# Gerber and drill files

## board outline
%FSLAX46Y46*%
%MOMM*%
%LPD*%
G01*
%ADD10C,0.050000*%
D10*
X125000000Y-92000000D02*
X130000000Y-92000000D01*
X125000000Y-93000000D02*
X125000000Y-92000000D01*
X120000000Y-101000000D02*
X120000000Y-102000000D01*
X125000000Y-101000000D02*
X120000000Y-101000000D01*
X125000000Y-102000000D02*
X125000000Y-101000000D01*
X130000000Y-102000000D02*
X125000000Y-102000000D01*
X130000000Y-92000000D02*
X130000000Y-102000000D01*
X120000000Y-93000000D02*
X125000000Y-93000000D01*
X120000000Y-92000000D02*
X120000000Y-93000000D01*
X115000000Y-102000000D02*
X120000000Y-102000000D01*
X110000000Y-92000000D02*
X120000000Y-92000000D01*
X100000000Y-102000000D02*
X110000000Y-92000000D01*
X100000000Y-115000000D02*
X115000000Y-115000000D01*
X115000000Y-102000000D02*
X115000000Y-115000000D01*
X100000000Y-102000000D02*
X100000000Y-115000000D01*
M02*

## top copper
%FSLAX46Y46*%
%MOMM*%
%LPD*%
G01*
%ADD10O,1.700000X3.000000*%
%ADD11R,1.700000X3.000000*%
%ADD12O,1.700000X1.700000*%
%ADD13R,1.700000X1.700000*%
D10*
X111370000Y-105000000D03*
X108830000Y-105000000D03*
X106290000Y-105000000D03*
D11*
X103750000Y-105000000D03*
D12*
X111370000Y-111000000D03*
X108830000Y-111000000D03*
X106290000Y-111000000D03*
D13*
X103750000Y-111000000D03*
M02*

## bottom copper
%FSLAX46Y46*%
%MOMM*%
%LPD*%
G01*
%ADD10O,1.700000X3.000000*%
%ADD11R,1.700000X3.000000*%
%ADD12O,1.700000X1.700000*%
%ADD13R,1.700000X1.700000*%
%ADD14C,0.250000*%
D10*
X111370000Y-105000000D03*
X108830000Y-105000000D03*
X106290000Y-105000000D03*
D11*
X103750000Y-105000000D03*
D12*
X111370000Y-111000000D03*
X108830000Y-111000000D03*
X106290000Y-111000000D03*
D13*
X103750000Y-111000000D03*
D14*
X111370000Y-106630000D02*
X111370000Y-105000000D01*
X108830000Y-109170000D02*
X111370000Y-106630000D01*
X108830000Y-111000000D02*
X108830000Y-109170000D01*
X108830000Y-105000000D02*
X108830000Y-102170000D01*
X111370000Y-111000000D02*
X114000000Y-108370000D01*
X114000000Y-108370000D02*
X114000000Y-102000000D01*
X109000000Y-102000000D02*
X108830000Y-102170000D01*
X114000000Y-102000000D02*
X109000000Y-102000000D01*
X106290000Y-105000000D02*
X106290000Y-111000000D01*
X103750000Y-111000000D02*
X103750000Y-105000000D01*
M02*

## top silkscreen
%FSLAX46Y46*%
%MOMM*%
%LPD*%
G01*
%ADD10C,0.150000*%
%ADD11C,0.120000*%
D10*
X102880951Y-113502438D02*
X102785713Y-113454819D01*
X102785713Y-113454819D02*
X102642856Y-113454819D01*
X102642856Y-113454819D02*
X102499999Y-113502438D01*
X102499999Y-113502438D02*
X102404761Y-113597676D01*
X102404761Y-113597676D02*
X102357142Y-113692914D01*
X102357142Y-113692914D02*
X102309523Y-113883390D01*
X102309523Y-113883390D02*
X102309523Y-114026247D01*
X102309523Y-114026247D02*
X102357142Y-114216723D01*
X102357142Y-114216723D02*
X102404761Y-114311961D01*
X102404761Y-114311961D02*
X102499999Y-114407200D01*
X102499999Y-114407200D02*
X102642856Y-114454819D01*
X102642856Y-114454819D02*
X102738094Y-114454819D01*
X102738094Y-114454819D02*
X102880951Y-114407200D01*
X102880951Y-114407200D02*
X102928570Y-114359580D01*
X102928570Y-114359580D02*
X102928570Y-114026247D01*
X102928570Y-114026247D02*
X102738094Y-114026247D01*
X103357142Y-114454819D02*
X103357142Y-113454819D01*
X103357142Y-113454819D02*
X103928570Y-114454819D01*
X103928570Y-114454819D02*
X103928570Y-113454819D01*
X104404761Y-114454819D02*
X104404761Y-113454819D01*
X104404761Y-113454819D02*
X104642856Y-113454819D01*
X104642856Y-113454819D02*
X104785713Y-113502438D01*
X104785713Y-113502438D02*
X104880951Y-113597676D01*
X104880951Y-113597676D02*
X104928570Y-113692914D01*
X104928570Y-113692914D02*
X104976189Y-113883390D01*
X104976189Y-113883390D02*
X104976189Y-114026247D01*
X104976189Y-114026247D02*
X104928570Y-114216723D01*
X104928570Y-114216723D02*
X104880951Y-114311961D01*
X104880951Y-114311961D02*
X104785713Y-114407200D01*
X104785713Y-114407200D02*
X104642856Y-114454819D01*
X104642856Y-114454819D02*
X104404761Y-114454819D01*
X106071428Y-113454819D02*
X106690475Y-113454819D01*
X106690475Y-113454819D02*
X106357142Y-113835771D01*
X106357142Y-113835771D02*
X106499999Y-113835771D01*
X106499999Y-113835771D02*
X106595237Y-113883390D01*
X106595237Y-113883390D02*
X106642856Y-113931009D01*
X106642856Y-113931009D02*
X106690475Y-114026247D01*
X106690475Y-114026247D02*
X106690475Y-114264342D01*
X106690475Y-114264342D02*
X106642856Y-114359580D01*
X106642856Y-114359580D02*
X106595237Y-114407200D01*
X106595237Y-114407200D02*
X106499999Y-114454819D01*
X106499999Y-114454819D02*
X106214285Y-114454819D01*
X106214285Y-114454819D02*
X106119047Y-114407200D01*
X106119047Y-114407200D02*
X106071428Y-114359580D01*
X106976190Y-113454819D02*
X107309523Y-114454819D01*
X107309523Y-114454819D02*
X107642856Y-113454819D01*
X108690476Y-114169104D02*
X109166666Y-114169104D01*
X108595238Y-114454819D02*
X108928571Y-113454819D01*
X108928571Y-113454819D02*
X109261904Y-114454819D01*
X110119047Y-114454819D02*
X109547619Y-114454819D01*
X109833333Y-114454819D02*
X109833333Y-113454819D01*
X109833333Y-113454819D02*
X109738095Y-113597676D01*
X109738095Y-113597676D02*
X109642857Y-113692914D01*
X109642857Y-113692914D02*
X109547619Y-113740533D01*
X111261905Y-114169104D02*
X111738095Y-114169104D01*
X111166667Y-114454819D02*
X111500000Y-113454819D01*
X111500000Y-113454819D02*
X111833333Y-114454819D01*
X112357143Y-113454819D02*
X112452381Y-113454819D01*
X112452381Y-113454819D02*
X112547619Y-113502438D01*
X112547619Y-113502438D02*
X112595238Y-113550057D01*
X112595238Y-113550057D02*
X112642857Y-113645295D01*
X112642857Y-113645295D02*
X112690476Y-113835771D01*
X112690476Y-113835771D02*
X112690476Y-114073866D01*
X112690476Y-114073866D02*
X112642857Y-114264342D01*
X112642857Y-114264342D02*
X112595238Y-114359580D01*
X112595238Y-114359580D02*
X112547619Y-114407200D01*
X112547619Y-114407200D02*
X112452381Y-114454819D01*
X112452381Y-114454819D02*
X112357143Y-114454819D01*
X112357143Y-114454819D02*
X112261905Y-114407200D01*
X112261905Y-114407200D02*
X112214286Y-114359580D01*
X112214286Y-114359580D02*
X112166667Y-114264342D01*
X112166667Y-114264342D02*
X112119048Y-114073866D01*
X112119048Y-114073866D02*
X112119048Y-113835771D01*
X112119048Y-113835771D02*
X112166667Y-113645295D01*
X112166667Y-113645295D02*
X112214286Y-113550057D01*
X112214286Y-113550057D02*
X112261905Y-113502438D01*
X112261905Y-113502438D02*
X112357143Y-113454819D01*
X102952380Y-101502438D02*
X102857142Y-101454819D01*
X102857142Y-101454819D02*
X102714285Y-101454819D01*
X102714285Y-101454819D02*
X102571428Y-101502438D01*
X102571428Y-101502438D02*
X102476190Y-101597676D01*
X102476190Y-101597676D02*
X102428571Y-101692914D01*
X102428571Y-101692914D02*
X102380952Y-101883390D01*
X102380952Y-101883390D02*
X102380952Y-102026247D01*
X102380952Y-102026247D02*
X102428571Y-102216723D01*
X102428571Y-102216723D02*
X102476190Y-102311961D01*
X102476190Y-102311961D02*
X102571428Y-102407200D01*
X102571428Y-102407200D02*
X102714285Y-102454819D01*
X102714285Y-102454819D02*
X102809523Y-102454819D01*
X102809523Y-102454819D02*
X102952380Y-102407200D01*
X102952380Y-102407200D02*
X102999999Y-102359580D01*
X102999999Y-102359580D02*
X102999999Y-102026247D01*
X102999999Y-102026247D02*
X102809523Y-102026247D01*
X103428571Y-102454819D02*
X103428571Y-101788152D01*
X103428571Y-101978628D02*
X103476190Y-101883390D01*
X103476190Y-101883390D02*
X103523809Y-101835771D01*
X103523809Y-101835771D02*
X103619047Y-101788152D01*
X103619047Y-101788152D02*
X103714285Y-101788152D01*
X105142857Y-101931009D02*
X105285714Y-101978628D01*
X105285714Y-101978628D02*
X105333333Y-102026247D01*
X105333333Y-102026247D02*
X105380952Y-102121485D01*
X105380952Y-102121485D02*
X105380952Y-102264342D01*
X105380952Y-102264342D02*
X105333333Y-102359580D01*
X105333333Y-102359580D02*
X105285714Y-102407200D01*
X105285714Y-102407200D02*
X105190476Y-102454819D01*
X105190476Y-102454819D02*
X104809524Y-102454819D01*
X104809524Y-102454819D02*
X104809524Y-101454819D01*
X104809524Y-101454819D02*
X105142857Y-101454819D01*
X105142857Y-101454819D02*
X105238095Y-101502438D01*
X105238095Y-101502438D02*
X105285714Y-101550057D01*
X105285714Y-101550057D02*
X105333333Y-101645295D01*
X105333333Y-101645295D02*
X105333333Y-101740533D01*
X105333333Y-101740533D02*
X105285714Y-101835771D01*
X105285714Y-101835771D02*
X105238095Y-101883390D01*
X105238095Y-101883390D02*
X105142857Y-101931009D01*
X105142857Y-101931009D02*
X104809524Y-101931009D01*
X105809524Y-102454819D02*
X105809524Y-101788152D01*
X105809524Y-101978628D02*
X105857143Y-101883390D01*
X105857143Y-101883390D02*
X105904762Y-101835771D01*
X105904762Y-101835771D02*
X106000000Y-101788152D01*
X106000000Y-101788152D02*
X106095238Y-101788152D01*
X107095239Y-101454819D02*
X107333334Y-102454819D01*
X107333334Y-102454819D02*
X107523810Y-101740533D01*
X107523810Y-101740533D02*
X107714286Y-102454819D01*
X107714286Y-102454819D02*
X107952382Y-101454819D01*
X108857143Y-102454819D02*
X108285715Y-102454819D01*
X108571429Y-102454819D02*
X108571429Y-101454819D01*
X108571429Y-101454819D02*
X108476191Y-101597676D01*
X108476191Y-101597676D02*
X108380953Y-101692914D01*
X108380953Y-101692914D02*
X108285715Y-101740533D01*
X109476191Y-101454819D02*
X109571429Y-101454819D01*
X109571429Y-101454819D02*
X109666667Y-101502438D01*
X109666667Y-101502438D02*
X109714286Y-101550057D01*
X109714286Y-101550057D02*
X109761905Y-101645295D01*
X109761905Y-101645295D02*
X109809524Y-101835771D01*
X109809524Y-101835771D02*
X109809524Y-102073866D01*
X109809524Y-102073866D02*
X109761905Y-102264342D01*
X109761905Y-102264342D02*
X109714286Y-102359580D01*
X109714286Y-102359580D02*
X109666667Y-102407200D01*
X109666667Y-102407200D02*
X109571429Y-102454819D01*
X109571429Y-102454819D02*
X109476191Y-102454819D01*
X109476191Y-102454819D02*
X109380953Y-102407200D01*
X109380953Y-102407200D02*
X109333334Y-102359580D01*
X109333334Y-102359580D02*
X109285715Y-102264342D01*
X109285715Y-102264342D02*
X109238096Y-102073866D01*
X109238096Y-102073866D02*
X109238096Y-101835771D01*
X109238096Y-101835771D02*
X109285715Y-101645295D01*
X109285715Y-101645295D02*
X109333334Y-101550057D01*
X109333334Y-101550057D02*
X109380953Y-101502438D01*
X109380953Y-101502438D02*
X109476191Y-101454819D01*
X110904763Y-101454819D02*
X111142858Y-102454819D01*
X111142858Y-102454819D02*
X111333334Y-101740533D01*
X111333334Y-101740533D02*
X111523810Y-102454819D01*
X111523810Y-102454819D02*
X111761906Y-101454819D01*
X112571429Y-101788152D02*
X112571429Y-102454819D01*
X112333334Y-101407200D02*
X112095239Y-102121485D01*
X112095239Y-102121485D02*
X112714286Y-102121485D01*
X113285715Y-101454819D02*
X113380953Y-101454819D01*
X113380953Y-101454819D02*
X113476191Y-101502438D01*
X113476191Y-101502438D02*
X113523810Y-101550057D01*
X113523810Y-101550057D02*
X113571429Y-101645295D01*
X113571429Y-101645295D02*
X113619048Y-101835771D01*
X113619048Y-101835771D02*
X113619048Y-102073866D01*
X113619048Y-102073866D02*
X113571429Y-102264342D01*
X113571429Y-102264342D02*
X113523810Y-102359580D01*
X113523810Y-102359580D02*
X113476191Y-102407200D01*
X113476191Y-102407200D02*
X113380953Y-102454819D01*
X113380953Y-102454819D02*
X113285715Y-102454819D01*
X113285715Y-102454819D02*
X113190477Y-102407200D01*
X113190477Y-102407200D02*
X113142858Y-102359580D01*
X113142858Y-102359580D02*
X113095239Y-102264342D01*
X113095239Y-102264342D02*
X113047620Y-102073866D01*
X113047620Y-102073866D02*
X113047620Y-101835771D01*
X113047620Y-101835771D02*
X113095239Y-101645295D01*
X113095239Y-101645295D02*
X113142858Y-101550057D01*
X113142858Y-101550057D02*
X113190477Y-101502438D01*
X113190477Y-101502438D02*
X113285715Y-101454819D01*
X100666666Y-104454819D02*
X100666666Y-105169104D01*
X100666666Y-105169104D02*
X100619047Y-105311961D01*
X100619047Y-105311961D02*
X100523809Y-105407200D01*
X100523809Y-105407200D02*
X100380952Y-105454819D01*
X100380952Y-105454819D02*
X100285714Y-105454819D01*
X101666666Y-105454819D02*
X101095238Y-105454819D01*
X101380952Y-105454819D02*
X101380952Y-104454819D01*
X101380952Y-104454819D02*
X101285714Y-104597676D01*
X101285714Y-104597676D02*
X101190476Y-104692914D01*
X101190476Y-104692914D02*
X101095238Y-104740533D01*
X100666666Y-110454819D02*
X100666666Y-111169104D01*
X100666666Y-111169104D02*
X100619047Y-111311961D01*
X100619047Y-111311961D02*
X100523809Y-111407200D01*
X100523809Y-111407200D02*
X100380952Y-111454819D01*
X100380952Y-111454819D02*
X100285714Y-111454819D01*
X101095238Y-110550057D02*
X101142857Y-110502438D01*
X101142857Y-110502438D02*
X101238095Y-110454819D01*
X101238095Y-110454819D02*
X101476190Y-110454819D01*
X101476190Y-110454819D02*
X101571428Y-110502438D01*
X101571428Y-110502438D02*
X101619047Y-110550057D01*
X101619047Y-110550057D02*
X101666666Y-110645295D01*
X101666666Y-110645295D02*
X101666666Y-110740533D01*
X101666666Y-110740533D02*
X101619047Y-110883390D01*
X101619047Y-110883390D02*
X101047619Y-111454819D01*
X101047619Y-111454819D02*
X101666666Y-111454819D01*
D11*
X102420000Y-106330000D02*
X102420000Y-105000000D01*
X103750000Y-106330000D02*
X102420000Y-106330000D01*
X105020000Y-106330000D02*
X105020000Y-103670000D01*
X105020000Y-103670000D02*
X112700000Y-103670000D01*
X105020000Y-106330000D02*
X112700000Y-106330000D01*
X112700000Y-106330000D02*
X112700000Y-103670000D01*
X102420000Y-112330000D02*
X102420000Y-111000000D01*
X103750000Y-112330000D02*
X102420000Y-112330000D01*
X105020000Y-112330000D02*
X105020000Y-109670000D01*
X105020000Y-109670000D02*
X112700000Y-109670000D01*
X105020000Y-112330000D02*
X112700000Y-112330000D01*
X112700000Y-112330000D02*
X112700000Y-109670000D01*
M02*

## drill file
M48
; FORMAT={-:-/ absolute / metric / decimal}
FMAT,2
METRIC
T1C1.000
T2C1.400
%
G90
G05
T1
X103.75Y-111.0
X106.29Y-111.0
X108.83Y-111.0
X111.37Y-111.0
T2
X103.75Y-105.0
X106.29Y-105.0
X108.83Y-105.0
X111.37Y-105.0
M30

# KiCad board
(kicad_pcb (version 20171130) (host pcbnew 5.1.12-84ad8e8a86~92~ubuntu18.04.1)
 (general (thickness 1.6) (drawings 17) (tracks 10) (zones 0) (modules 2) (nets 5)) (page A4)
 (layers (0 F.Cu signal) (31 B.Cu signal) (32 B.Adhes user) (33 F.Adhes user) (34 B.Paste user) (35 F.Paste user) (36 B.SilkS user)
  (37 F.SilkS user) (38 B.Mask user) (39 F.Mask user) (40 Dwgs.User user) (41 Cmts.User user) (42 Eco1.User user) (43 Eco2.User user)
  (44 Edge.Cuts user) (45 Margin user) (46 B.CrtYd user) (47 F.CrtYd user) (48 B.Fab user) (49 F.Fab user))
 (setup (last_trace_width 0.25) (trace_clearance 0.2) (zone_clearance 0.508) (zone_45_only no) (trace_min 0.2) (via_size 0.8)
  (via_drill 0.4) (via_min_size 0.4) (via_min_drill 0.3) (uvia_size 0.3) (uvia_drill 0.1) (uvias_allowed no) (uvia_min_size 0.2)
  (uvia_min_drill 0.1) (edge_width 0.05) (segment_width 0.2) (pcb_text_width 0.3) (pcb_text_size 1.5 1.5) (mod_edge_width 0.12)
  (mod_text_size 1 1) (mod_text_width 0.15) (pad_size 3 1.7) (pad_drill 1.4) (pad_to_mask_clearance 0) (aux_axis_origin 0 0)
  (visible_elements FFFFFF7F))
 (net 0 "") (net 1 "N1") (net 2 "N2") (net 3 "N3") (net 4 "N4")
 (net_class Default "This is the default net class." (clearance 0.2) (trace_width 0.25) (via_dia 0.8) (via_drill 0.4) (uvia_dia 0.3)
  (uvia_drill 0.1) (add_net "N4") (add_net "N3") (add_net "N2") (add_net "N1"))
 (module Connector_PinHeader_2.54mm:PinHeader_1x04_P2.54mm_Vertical (layer F.Cu) (at 103.75 105 90)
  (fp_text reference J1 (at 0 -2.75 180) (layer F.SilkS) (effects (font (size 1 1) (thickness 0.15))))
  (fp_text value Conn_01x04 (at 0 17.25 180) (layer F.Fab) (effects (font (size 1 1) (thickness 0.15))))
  (fp_line (start -1.33 -1.33) (end 0 -1.33) (layer F.SilkS) (width 0.12))
  (fp_line (start -1.33 0) (end -1.33 -1.33) (layer F.SilkS) (width 0.12))
  (fp_line (start -1.33 1.27) (end 1.33 1.27) (layer F.SilkS) (width 0.12))
  (fp_line (start 1.33 1.27) (end 1.33 8.95) (layer F.SilkS) (width 0.12))
  (fp_line (start -1.33 1.27) (end -1.33 8.95) (layer F.SilkS) (width 0.12))
  (fp_line (start -1.33 8.95) (end 1.33 8.95) (layer F.SilkS) (width 0.12))
  (pad 4 thru_hole oval (at 0 7.62 90) (size 3 1.7) (drill 1.4) (layers *.Cu *.Mask) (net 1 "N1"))
  (pad 3 thru_hole oval (at 0 5.08 90) (size 3 1.7) (drill 1.4) (layers *.Cu *.Mask) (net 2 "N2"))
  (pad 2 thru_hole oval (at 0 2.54 90) (size 3 1.7) (drill 1.4) (layers *.Cu *.Mask) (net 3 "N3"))
  (pad 1 thru_hole rect (at 0 0 90) (size 3 1.7) (drill 1.4) (layers *.Cu *.Mask) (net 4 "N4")))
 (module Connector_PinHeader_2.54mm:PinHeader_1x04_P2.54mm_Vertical (layer F.Cu) (at 103.75 111 90)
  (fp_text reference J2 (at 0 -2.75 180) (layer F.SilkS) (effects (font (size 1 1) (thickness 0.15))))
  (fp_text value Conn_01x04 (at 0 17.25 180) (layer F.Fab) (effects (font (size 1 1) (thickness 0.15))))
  (fp_line (start -1.33 -1.33) (end 0 -1.33) (layer F.SilkS) (width 0.12))
  (fp_line (start -1.33 0) (end -1.33 -1.33) (layer F.SilkS) (width 0.12))
  (fp_line (start -1.33 1.27) (end 1.33 1.27) (layer F.SilkS) (width 0.12))
  (fp_line (start 1.33 1.27) (end 1.33 8.95) (layer F.SilkS) (width 0.12))
  (fp_line (start -1.33 1.27) (end -1.33 8.95) (layer F.SilkS) (width 0.12))
  (fp_line (start -1.33 8.95) (end 1.33 8.95) (layer F.SilkS) (width 0.12))
  (pad 4 thru_hole oval (at 0 7.62 90) (size 1.7 1.7) (drill 1) (layers *.Cu *.Mask) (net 2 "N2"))
  (pad 3 thru_hole oval (at 0 5.08 90) (size 1.7 1.7) (drill 1) (layers *.Cu *.Mask) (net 1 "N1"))
  (pad 2 thru_hole oval (at 0 2.54 90) (size 1.7 1.7) (drill 1) (layers *.Cu *.Mask) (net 3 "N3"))
  (pad 1 thru_hole rect (at 0 0 90) (size 1.7 1.7) (drill 1) (layers *.Cu *.Mask) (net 4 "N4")))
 (gr_line (start 125 92) (end 130 92) (layer Edge.Cuts) (width 0.05))
 (gr_line (start 125 93) (end 125 92) (layer Edge.Cuts) (width 0.05))
 (gr_line (start 120 101) (end 120 102) (layer Edge.Cuts) (width 0.05))
 (gr_line (start 125 101) (end 120 101) (layer Edge.Cuts) (width 0.05))
 (gr_line (start 125 102) (end 125 101) (layer Edge.Cuts) (width 0.05))
 (gr_line (start 130 102) (end 125 102) (layer Edge.Cuts) (width 0.05))
 (gr_line (start 130 92) (end 130 102) (layer Edge.Cuts) (width 0.05))
 (gr_line (start 120 93) (end 125 93) (layer Edge.Cuts) (width 0.05))
 (gr_line (start 120 92) (end 120 93) (layer Edge.Cuts) (width 0.05))
 (gr_line (start 115 102) (end 120 102) (layer Edge.Cuts) (width 0.05))
 (gr_line (start 110 92) (end 120 92) (layer Edge.Cuts) (width 0.05))
 (gr_line (start 100 102) (end 110 92) (layer Edge.Cuts) (width 0.05))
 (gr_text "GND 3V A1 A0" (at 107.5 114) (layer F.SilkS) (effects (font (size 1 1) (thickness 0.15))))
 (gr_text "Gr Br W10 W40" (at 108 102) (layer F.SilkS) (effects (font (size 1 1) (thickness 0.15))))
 (gr_line (start 100 115) (end 115 115) (layer Edge.Cuts) (width 0.05))
 (gr_line (start 115 102) (end 115 115) (layer Edge.Cuts) (width 0.05))
 (gr_line (start 100 102) (end 100 115) (layer Edge.Cuts) (width 0.05))
 (segment (start 111.37 106.63) (end 111.37 105) (width 0.25) (layer B.Cu) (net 1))
 (segment (start 108.83 109.17) (end 111.37 106.63) (width 0.25) (layer B.Cu) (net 1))
 (segment (start 108.83 111) (end 108.83 109.17) (width 0.25) (layer B.Cu) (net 1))
 (segment (start 108.83 105) (end 108.83 102.17) (width 0.25) (layer B.Cu) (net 2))
 (segment (start 111.37 111) (end 114 108.37) (width 0.25) (layer B.Cu) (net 2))
 (segment (start 114 108.37) (end 114 102) (width 0.25) (layer B.Cu) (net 2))
 (segment (start 109 102) (end 108.83 102.17) (width 0.25) (layer B.Cu) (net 2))
 (segment (start 114 102) (end 109 102) (width 0.25) (layer B.Cu) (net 2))
 (segment (start 106.29 105) (end 106.29 111) (width 0.25) (layer B.Cu) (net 3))
 (segment (start 103.75 111) (end 103.75 105) (width 0.25) (layer B.Cu) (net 4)))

